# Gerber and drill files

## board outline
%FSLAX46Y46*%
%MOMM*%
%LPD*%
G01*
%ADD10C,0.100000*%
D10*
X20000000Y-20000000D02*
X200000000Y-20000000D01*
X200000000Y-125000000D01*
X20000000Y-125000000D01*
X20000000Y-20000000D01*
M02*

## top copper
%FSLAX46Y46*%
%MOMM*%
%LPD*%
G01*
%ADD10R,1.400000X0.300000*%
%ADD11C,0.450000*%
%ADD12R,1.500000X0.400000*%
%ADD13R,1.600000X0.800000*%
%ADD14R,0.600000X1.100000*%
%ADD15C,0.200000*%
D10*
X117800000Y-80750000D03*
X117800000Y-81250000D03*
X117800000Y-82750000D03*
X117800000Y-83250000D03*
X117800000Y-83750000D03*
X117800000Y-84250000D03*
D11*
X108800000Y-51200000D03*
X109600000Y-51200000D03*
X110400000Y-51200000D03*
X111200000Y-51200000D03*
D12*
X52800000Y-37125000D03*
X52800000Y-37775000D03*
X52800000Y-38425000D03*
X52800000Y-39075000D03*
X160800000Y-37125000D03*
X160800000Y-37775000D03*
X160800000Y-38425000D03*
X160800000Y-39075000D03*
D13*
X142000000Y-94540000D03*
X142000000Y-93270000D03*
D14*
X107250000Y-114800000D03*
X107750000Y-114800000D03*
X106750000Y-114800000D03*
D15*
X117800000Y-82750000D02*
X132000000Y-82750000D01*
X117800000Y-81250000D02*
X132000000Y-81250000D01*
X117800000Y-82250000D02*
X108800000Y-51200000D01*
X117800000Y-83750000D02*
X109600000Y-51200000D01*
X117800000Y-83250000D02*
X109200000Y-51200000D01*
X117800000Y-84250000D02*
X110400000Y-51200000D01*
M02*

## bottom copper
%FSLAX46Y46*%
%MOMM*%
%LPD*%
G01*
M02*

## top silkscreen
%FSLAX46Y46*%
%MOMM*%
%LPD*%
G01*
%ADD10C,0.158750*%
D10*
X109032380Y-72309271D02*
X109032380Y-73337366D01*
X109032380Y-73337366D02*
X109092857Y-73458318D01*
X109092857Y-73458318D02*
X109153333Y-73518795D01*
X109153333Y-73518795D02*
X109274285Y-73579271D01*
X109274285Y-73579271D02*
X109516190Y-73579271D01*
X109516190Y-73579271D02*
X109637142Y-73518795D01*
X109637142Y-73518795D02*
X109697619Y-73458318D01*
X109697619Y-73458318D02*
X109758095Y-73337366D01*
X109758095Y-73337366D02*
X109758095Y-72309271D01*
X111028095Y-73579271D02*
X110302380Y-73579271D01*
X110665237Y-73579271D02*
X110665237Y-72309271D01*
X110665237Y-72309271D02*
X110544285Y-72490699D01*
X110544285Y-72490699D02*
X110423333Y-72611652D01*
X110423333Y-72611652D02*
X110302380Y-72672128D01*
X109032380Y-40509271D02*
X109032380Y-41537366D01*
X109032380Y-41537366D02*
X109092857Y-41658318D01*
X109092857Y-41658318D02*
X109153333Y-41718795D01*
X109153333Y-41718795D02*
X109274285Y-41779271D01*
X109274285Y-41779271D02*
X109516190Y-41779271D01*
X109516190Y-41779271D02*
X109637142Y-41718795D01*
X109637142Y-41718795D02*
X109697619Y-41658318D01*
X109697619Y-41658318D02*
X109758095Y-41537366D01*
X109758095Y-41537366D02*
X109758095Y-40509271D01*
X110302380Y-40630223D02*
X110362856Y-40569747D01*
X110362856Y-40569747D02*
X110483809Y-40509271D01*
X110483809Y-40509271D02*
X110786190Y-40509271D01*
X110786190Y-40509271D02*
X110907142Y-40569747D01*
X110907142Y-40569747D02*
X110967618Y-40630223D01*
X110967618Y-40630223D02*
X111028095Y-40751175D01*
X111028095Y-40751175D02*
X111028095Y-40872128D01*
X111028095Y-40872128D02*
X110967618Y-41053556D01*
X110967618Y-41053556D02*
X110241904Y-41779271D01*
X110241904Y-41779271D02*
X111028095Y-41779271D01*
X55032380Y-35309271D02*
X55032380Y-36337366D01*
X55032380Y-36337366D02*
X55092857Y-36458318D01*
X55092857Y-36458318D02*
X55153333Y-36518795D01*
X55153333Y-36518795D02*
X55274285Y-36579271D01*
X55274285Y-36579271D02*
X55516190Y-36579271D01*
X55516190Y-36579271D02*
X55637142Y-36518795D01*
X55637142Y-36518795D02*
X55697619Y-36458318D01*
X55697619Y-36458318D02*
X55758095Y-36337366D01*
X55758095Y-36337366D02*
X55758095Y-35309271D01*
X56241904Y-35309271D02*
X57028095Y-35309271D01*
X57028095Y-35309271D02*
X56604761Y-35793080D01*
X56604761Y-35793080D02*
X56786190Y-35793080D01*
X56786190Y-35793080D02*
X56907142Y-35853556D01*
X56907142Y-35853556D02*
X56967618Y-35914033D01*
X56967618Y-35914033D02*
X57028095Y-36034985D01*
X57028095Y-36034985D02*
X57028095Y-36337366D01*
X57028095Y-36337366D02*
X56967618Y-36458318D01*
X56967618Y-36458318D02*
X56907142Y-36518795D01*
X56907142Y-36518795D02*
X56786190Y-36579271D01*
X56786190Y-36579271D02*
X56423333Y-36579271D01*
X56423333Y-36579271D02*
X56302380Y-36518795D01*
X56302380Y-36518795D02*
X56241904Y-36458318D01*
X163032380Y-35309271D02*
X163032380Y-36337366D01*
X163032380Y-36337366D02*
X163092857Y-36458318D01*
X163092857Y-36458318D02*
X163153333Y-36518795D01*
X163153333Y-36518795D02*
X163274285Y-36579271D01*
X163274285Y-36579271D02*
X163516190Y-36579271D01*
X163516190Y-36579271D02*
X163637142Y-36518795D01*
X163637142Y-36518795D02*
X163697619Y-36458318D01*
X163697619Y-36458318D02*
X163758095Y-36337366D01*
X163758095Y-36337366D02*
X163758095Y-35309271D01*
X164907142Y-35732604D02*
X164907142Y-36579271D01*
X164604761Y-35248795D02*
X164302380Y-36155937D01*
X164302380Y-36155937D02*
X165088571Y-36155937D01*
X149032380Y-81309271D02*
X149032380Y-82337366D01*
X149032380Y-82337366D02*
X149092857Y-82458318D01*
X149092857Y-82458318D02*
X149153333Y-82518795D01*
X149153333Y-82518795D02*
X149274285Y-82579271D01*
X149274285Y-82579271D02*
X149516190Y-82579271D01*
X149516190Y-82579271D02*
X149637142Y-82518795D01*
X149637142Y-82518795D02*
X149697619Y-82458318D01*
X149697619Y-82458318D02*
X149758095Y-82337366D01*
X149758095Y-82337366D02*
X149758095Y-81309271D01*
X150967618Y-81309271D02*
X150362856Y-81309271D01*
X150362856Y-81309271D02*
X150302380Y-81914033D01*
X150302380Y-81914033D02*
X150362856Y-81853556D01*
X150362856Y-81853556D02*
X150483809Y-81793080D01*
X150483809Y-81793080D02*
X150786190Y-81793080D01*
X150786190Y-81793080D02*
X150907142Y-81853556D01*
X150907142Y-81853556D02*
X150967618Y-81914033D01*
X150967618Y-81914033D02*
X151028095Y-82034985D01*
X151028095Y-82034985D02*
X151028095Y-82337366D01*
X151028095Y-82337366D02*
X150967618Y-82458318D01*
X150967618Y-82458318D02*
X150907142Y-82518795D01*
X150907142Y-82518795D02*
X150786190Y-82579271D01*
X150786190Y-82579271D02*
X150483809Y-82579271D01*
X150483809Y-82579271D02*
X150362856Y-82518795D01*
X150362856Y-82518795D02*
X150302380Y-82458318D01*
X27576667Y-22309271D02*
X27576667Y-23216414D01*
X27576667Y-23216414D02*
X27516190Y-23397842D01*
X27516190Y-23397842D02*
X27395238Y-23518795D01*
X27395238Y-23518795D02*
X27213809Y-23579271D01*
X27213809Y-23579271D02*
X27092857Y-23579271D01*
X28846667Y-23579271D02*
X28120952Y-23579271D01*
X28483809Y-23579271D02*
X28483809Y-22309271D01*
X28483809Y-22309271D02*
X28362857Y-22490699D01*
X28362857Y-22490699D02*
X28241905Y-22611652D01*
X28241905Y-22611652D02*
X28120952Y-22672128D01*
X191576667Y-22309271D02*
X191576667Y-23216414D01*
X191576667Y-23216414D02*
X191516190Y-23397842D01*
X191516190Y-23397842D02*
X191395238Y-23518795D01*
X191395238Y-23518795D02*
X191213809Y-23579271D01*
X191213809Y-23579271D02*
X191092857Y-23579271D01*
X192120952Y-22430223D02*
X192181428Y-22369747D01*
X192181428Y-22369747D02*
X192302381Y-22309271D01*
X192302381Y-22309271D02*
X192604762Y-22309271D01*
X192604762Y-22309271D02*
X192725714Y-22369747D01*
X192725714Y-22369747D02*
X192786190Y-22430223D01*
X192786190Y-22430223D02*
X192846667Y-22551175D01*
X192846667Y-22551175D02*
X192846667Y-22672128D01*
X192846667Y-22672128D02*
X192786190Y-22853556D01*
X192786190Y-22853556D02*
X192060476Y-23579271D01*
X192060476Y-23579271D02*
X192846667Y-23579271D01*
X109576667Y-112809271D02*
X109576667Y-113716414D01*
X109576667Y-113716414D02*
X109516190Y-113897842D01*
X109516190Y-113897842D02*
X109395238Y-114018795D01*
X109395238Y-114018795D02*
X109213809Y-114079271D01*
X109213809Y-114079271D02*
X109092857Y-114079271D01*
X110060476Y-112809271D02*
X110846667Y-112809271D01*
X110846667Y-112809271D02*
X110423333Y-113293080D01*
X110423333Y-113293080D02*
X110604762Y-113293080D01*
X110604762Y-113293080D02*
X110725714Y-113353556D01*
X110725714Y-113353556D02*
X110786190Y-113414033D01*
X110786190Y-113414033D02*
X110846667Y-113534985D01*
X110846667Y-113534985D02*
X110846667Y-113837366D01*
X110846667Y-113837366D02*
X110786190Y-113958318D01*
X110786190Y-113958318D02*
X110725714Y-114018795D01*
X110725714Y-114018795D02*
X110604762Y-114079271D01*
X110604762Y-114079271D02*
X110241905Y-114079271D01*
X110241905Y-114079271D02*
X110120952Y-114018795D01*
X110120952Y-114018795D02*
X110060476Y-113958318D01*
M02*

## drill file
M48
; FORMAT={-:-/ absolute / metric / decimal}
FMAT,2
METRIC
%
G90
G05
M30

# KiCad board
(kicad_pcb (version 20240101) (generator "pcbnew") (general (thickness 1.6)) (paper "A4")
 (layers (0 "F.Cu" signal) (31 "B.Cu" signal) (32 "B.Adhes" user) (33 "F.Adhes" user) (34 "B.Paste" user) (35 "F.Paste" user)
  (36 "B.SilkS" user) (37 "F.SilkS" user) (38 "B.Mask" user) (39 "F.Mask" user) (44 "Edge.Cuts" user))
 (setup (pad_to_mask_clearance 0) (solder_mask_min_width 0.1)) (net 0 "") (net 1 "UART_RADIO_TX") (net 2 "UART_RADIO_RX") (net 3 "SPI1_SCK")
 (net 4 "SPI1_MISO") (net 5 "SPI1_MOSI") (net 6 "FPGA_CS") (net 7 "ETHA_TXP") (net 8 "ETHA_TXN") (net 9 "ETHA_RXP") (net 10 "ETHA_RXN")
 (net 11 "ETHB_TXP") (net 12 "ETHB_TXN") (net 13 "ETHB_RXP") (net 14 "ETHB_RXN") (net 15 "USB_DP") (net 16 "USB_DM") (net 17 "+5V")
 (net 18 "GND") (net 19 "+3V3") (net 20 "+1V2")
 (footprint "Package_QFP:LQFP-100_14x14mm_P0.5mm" (layer "F.Cu") (at 110 82) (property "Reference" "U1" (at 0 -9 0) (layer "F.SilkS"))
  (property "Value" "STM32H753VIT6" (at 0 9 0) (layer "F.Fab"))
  (pad "57" smd rect (at 7.8 -1.25) (size 1.4 0.3) (layers "F.Cu" "F.Paste" "F.Mask") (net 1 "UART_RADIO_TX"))
  (pad "58" smd rect (at 7.8 -0.75) (size 1.4 0.3) (layers "F.Cu" "F.Paste" "F.Mask") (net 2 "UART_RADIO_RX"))
  (pad "61" smd rect (at 7.8 0.75) (size 1.4 0.3) (layers "F.Cu" "F.Paste" "F.Mask") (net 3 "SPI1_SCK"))
  (pad "62" smd rect (at 7.8 1.25) (size 1.4 0.3) (layers "F.Cu" "F.Paste" "F.Mask") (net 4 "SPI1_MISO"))
  (pad "63" smd rect (at 7.8 1.75) (size 1.4 0.3) (layers "F.Cu" "F.Paste" "F.Mask") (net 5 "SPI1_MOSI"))
  (pad "64" smd rect (at 7.8 2.25) (size 1.4 0.3) (layers "F.Cu" "F.Paste" "F.Mask") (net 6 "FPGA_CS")))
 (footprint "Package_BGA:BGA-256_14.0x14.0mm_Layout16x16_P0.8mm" (layer "F.Cu") (at 110 50)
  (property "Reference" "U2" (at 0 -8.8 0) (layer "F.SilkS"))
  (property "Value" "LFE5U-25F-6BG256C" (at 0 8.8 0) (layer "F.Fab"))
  (pad "D7" smd circle (at -1.2 1.2) (size 0.45 0.45) (layers "F.Cu" "F.Mask") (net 3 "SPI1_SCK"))
  (pad "D8" smd circle (at -0.4 1.2) (size 0.45 0.45) (layers "F.Cu" "F.Mask") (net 5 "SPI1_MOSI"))
  (pad "D9" smd circle (at 0.4 1.2) (size 0.45 0.45) (layers "F.Cu" "F.Mask") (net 4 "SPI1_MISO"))
  (pad "D10" smd circle (at 1.2 1.2) (size 0.45 0.45) (layers "F.Cu" "F.Mask") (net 6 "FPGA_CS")))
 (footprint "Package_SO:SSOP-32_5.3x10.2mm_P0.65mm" (layer "F.Cu") (at 56 42) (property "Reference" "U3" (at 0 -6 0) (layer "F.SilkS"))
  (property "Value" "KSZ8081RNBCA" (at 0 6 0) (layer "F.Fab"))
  (pad "1" smd rect (at -3.2 -4.875) (size 1.5 0.4) (layers "F.Cu" "F.Paste" "F.Mask") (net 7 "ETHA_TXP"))
  (pad "2" smd rect (at -3.2 -4.225) (size 1.5 0.4) (layers "F.Cu" "F.Paste" "F.Mask") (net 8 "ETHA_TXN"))
  (pad "3" smd rect (at -3.2 -3.575) (size 1.5 0.4) (layers "F.Cu" "F.Paste" "F.Mask") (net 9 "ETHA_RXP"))
  (pad "4" smd rect (at -3.2 -2.925) (size 1.5 0.4) (layers "F.Cu" "F.Paste" "F.Mask") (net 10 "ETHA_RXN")))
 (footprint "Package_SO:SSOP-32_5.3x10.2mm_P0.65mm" (layer "F.Cu") (at 164 42) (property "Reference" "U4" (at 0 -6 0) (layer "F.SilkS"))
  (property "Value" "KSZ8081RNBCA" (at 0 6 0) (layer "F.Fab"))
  (pad "1" smd rect (at -3.2 -4.875) (size 1.5 0.4) (layers "F.Cu" "F.Paste" "F.Mask") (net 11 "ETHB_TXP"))
  (pad "2" smd rect (at -3.2 -4.225) (size 1.5 0.4) (layers "F.Cu" "F.Paste" "F.Mask") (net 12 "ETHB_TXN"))
  (pad "3" smd rect (at -3.2 -3.575) (size 1.5 0.4) (layers "F.Cu" "F.Paste" "F.Mask") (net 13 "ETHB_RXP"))
  (pad "4" smd rect (at -3.2 -2.925) (size 1.5 0.4) (layers "F.Cu" "F.Paste" "F.Mask") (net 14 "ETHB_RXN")))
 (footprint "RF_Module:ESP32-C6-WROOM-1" (layer "F.Cu") (at 150 92) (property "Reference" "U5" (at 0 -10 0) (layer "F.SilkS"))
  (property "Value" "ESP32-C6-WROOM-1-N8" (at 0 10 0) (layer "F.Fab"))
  (pad "16" smd rect (at -8 2.54) (size 1.6 0.8) (layers "F.Cu" "F.Paste" "F.Mask") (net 1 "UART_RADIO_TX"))
  (pad "17" smd rect (at -8 1.27) (size 1.6 0.8) (layers "F.Cu" "F.Paste" "F.Mask") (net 2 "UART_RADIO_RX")))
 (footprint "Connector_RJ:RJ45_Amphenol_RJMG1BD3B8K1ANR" (layer "F.Cu") (at 28 34)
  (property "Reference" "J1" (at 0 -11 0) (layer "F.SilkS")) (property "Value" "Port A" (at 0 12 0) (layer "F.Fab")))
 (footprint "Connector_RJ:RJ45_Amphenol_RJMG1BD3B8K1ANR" (layer "F.Cu") (at 192 34)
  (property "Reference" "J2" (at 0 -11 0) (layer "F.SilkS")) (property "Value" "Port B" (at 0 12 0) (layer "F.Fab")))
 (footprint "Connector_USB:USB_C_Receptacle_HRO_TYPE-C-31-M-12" (layer "F.Cu") (at 110 118)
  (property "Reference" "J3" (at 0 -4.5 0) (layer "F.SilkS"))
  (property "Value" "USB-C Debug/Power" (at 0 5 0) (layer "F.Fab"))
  (pad "A6" smd rect (at -2.75 -3.2) (size 0.6 1.1) (layers "F.Cu" "F.Paste" "F.Mask") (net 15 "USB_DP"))
  (pad "A7" smd rect (at -2.25 -3.2) (size 0.6 1.1) (layers "F.Cu" "F.Paste" "F.Mask") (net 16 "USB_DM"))
  (pad "A4" smd rect (at -3.25 -3.2) (size 0.6 1.1) (layers "F.Cu" "F.Paste" "F.Mask") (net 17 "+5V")))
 (gr_rect (start 20 20) (end 200 125) (stroke (width 0.1) (type default)) (fill none) (layer "Edge.Cuts"))
 (segment (start 117.8 82.75) (end 132 82.75) (width 0.2) (layer "F.Cu") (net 1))
 (segment (start 117.8 81.25) (end 132 81.25) (width 0.2) (layer "F.Cu") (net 2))
 (segment (start 117.8 82.25) (end 108.8 51.2) (width 0.2) (layer "F.Cu") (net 3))
 (segment (start 117.8 83.75) (end 109.6 51.2) (width 0.2) (layer "F.Cu") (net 4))
 (segment (start 117.8 83.25) (end 109.2 51.2) (width 0.2) (layer "F.Cu") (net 5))
 (segment (start 117.8 84.25) (end 110.4 51.2) (width 0.2) (layer "F.Cu") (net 6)))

